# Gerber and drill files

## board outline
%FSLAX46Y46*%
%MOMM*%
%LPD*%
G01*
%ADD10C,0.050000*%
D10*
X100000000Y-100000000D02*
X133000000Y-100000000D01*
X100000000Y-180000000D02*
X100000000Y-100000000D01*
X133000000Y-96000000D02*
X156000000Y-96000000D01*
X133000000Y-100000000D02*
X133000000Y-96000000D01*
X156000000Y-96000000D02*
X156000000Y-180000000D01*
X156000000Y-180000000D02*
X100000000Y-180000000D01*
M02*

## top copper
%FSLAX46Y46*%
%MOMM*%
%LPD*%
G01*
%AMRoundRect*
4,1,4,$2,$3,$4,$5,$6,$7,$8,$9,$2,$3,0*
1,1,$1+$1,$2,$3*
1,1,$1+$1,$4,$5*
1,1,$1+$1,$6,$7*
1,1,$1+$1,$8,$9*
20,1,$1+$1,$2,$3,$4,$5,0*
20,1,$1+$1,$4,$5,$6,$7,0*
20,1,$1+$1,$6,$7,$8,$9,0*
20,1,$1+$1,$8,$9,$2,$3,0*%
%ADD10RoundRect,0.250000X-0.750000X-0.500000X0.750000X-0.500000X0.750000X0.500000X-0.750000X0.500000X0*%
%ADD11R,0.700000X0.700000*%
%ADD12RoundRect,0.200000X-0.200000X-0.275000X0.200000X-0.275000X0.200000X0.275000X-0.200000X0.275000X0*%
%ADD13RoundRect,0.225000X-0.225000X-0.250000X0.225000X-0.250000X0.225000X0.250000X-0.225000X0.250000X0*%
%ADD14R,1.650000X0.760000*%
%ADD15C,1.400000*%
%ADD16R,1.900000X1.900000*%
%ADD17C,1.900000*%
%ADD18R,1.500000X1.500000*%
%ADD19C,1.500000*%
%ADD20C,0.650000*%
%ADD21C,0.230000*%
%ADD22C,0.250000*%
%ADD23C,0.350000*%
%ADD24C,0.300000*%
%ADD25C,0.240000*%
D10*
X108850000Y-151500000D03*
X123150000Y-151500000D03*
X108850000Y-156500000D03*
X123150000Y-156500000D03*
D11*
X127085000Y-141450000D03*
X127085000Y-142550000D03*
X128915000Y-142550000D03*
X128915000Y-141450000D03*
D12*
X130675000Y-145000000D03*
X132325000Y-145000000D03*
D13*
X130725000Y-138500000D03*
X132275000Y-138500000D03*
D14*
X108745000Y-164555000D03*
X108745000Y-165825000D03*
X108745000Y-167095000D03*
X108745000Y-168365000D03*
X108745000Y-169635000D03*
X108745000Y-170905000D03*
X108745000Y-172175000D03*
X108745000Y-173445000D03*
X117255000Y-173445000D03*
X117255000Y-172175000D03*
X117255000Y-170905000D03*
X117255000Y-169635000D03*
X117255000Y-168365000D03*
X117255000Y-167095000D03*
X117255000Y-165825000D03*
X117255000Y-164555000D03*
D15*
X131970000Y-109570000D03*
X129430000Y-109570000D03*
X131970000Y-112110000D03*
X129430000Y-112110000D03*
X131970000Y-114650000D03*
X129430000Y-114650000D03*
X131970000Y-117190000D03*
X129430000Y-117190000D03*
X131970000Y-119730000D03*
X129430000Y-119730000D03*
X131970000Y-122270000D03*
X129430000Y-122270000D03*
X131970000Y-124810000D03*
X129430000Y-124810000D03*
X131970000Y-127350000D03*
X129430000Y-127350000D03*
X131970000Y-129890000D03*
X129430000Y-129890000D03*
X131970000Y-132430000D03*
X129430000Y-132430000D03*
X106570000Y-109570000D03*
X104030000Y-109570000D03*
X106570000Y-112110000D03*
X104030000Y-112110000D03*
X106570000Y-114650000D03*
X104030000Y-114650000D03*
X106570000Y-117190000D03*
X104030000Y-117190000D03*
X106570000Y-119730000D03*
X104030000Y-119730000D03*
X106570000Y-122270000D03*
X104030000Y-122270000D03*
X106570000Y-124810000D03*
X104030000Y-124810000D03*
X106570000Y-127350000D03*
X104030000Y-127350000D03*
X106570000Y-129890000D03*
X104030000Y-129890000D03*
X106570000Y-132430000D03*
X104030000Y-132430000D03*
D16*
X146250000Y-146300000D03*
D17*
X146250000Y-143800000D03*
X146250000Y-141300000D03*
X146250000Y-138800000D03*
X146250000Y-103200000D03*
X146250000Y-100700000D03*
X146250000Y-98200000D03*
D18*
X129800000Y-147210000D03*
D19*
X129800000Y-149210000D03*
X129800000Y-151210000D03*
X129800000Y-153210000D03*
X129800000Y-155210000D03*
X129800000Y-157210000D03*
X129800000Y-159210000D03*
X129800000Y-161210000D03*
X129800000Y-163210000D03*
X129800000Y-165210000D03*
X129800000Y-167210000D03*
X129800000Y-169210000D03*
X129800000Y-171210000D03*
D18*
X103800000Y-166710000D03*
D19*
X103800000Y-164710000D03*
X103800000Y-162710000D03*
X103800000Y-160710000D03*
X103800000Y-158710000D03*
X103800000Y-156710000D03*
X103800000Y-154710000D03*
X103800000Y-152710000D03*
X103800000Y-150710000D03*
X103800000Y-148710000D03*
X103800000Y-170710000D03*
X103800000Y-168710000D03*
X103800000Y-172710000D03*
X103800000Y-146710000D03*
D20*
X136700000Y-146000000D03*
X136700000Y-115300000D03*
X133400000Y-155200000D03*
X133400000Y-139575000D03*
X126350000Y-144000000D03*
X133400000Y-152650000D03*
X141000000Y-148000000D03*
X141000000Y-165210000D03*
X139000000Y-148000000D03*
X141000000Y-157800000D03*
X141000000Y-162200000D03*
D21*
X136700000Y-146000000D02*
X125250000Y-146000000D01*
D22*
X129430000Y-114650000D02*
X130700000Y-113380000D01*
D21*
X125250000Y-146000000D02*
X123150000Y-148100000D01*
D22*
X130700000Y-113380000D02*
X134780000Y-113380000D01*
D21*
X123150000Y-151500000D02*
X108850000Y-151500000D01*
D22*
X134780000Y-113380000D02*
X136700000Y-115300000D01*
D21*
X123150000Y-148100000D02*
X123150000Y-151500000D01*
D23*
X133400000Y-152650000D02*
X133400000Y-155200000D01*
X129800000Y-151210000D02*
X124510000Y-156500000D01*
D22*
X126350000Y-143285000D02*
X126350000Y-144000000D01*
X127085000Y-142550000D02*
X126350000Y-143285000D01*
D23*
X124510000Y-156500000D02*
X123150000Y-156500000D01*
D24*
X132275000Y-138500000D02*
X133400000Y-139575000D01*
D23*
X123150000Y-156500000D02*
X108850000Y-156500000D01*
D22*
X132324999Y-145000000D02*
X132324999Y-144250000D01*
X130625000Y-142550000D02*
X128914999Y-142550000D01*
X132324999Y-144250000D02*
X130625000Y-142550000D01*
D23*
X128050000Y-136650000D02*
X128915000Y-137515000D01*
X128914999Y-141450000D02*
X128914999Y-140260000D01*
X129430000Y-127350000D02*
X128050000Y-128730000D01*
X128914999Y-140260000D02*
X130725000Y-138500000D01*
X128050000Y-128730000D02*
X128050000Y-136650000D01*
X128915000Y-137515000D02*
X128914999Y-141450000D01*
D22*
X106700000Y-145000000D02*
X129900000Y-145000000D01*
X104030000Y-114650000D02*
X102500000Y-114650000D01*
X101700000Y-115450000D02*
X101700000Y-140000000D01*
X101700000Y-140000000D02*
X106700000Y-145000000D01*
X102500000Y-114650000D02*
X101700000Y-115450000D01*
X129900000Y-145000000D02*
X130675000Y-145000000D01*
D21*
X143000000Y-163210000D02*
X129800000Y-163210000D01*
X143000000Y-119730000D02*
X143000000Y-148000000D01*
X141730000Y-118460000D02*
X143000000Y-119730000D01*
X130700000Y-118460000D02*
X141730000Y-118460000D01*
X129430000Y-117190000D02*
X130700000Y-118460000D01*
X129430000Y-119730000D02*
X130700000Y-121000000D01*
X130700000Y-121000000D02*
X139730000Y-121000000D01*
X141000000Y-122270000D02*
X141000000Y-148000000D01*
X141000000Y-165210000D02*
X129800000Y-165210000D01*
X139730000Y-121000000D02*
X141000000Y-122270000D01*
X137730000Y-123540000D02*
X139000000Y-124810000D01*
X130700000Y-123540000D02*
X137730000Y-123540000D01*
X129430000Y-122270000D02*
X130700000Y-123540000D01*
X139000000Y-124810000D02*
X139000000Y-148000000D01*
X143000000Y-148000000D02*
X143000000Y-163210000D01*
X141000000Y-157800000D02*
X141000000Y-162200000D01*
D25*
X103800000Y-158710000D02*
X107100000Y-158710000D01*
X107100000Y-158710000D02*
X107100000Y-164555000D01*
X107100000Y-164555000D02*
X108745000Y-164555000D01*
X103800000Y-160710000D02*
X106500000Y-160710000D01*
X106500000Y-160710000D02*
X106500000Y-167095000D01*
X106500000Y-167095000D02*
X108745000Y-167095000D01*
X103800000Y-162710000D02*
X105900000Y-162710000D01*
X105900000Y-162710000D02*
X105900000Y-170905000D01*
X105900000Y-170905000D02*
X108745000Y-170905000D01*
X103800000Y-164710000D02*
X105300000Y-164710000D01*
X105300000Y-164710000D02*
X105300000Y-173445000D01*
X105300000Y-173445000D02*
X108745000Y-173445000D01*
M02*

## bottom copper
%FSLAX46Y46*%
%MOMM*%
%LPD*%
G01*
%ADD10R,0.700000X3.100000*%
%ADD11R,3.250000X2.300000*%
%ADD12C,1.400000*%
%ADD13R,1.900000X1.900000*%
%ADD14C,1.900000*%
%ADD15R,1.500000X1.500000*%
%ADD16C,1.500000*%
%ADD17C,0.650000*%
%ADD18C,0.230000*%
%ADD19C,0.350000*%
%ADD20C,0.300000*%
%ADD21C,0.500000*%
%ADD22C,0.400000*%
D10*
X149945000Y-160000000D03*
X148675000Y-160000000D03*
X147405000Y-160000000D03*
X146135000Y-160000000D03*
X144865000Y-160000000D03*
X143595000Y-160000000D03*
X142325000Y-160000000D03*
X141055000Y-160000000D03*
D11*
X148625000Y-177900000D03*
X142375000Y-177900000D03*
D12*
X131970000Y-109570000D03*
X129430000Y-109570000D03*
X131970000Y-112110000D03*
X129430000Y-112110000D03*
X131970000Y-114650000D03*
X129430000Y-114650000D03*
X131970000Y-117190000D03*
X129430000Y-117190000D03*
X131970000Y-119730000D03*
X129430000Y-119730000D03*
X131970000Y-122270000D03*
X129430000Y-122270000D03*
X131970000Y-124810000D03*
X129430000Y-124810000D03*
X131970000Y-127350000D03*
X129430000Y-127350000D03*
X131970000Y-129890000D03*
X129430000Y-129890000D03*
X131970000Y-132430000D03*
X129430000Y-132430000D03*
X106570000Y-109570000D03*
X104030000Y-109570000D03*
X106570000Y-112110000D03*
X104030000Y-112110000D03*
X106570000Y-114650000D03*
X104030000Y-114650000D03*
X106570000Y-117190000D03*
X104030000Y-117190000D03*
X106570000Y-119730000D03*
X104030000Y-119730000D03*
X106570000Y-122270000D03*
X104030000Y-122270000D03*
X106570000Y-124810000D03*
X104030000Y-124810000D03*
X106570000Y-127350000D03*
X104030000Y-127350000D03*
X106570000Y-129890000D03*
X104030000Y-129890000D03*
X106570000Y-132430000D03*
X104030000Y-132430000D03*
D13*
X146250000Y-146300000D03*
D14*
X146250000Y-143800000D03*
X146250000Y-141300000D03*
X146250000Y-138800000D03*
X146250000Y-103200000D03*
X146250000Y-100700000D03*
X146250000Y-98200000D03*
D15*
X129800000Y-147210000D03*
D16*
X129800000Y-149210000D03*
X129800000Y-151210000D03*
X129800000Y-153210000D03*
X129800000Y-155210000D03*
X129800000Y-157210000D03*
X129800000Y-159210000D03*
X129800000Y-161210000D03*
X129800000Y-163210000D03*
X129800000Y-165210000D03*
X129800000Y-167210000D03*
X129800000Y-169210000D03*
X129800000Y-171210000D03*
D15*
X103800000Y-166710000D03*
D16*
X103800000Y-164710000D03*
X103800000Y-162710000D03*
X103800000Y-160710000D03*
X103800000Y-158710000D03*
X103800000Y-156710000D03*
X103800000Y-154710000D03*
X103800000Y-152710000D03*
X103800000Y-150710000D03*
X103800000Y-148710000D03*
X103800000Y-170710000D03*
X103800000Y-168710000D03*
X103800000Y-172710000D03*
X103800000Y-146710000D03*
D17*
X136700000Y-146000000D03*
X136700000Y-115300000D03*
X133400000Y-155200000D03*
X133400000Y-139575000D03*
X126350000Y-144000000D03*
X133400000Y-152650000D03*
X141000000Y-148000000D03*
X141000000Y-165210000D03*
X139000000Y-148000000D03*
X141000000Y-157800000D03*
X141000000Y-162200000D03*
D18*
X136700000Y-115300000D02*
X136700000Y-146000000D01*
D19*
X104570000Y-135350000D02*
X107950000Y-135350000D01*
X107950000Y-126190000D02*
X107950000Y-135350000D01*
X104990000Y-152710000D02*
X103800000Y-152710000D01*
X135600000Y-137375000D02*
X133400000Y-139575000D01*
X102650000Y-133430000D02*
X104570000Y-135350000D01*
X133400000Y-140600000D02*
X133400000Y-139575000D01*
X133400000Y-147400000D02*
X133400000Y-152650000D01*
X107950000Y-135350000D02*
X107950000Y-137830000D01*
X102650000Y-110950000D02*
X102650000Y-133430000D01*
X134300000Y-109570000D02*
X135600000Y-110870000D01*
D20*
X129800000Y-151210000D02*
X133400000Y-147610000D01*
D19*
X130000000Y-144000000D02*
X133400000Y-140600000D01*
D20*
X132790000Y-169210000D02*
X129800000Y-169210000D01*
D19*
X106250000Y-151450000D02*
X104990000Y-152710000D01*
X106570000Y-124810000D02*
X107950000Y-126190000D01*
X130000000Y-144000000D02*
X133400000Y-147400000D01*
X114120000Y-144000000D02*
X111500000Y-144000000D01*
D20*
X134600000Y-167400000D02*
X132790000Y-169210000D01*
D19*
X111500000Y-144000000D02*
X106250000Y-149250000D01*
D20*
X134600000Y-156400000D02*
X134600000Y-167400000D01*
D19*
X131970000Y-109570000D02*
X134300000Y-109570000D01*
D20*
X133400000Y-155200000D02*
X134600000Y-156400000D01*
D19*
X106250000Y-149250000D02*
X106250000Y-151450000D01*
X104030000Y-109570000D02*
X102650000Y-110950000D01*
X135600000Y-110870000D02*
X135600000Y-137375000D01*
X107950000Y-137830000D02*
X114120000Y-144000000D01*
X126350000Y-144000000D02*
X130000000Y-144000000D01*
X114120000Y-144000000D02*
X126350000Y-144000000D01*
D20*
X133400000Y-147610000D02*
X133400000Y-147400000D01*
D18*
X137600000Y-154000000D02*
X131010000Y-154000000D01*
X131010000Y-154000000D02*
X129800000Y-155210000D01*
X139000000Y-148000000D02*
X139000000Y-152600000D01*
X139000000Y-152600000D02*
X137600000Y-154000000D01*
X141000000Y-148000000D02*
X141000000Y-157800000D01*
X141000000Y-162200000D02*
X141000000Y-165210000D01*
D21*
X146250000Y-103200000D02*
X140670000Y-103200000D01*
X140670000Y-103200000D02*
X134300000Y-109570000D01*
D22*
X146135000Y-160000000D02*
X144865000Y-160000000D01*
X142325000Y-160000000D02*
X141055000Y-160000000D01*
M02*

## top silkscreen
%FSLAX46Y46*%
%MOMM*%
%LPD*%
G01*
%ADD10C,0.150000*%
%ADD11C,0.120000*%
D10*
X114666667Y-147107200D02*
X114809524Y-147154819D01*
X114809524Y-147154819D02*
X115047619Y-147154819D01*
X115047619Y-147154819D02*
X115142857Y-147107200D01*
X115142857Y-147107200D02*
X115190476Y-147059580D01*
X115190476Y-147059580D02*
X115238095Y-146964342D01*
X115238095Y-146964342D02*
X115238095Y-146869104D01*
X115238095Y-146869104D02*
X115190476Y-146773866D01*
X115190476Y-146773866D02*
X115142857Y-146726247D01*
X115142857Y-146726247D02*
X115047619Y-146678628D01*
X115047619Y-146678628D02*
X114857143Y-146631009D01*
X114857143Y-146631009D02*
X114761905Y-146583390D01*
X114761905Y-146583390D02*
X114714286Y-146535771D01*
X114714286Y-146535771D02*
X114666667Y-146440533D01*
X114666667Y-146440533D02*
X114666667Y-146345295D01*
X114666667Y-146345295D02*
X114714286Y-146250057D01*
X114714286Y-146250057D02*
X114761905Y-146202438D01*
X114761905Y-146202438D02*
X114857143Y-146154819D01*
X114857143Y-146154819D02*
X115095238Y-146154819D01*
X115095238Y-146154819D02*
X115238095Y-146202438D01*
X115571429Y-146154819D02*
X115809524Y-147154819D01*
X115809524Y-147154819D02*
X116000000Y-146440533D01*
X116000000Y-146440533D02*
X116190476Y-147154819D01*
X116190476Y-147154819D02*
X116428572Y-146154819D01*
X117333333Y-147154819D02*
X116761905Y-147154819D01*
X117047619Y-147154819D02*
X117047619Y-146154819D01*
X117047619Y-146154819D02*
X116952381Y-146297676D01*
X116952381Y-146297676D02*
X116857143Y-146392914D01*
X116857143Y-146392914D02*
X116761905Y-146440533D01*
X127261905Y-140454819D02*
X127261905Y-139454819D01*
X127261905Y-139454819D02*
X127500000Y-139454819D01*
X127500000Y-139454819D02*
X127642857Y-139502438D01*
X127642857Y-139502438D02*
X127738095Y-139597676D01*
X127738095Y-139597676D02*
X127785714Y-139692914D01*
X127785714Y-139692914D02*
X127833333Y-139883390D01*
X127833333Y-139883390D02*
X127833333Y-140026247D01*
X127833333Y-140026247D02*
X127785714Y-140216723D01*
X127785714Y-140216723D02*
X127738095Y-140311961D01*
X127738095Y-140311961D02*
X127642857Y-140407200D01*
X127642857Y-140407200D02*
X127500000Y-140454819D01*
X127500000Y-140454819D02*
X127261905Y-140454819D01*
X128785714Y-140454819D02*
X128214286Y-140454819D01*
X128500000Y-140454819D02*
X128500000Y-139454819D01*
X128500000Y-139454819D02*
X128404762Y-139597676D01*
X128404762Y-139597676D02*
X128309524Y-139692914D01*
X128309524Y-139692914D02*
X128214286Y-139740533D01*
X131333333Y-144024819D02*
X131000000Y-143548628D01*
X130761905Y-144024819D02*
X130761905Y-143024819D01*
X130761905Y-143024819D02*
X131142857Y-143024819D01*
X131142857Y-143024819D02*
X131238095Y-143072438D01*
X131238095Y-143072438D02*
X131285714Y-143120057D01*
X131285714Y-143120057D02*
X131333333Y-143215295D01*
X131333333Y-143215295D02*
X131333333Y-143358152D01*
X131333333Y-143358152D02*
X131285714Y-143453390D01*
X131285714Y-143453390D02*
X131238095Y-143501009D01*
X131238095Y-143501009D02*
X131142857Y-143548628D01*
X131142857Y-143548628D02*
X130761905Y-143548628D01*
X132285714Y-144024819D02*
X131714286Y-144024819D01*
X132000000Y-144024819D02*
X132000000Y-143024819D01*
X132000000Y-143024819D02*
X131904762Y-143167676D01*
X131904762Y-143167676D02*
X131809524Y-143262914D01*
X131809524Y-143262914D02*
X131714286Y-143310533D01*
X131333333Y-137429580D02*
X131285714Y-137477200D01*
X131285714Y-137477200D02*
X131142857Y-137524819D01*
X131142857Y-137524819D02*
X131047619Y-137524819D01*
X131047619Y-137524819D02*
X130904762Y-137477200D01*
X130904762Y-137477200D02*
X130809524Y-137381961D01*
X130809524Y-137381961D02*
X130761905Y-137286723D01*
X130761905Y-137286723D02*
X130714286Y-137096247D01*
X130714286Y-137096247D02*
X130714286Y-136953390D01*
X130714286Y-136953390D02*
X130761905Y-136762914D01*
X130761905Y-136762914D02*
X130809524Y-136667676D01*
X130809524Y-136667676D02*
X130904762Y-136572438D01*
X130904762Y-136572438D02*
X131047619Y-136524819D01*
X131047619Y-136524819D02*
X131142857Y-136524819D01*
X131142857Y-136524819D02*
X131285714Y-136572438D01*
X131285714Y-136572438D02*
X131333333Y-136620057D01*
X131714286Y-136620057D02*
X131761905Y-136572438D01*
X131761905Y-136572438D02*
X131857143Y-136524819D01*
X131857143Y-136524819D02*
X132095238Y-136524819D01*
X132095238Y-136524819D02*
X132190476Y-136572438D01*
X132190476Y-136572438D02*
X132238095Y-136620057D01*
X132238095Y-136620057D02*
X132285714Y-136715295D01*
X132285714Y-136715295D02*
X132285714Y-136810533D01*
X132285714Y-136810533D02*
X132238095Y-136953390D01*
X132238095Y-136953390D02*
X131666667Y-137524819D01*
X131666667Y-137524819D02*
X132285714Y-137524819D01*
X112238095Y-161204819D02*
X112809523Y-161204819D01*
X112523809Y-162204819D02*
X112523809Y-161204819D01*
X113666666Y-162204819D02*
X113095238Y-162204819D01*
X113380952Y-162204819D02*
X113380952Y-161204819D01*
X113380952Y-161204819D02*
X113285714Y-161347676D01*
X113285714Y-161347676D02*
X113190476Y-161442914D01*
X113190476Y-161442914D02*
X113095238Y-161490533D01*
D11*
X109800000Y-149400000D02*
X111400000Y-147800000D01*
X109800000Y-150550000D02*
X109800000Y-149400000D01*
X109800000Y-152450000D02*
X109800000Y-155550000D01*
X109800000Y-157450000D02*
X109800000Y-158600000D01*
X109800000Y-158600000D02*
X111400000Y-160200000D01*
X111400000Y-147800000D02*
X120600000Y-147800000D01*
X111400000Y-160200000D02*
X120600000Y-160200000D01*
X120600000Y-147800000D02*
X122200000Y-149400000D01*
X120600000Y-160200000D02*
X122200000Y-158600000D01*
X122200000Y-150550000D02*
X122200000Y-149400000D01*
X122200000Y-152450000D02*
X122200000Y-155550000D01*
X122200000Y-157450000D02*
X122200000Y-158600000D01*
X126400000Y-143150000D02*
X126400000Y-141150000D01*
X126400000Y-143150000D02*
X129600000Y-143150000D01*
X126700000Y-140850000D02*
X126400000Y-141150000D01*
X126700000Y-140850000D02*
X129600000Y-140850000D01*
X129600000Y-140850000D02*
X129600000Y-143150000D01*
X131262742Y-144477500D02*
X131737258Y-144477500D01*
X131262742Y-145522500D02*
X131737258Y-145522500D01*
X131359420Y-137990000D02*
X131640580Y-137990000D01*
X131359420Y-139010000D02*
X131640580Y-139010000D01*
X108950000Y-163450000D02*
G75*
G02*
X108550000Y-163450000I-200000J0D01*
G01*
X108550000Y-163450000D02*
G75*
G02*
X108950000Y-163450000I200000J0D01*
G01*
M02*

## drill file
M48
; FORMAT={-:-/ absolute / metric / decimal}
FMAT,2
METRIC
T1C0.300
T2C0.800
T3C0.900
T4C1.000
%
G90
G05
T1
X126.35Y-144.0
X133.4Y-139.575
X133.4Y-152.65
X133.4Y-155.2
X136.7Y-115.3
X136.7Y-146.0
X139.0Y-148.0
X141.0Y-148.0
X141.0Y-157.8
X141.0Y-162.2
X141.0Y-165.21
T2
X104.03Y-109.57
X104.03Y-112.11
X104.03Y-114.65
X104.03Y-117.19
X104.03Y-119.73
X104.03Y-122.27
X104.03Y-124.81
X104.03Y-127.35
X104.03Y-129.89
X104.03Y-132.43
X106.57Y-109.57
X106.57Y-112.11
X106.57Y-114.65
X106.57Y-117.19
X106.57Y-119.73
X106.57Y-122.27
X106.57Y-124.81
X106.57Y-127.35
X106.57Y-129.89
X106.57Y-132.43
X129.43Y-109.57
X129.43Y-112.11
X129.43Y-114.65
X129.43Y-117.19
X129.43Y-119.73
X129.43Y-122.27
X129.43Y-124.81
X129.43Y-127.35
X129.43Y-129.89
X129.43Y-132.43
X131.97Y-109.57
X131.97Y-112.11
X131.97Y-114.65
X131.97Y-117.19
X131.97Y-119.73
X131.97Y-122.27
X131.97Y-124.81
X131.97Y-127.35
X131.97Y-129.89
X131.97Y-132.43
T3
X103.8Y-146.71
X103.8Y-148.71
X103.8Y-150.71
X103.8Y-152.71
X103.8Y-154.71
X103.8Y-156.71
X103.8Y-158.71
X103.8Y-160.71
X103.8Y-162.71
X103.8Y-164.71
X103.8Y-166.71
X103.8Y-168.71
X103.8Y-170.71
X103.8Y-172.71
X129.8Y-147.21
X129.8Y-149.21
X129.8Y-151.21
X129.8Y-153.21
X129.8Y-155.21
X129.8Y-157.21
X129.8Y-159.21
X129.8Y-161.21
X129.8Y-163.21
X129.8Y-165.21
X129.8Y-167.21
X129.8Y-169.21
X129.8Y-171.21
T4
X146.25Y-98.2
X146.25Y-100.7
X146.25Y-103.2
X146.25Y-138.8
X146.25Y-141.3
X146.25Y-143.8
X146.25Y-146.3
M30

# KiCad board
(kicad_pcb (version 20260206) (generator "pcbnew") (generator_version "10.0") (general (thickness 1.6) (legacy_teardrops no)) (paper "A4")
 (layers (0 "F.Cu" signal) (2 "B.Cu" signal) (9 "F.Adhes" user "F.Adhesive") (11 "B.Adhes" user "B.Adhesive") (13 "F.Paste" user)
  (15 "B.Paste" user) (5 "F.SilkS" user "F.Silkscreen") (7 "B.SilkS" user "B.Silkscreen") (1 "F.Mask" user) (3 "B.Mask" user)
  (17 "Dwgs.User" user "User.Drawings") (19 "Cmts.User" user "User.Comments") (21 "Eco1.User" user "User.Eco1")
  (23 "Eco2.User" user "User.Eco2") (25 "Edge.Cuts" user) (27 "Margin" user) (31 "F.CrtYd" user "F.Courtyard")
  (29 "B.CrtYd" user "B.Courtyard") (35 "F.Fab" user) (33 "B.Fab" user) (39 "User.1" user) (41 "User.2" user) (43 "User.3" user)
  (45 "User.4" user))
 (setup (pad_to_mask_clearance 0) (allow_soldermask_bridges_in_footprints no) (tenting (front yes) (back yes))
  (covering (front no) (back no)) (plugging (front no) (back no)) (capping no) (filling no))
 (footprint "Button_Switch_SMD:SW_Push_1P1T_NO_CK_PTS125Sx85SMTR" (layer "F.Cu") (at 116 154)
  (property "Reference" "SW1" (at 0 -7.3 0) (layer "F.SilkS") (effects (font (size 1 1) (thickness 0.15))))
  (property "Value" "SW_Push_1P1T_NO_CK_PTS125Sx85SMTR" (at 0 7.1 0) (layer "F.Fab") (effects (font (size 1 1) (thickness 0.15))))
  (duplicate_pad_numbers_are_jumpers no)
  (fp_line (start -6.2 -4.6) (end -4.6 -6.2) (stroke (width 0.12) (type solid)) (layer "F.SilkS"))
  (fp_line (start -6.2 -3.45) (end -6.2 -4.6) (stroke (width 0.12) (type solid)) (layer "F.SilkS"))
  (fp_line (start -6.2 -1.55) (end -6.2 1.55) (stroke (width 0.12) (type solid)) (layer "F.SilkS"))
  (fp_line (start -6.2 3.45) (end -6.2 4.6) (stroke (width 0.12) (type solid)) (layer "F.SilkS"))
  (fp_line (start -6.2 4.6) (end -4.6 6.2) (stroke (width 0.12) (type solid)) (layer "F.SilkS"))
  (fp_line (start -4.6 -6.2) (end 4.6 -6.2) (stroke (width 0.12) (type solid)) (layer "F.SilkS"))
  (fp_line (start -4.6 6.2) (end 4.6 6.2) (stroke (width 0.12) (type solid)) (layer "F.SilkS"))
  (fp_line (start 4.6 -6.2) (end 6.2 -4.6) (stroke (width 0.12) (type solid)) (layer "F.SilkS"))
  (fp_line (start 4.6 6.2) (end 6.2 4.6) (stroke (width 0.12) (type solid)) (layer "F.SilkS"))
  (fp_line (start 6.2 -3.45) (end 6.2 -4.6) (stroke (width 0.12) (type solid)) (layer "F.SilkS"))
  (fp_line (start 6.2 -1.55) (end 6.2 1.55) (stroke (width 0.12) (type solid)) (layer "F.SilkS"))
  (fp_line (start 6.2 3.45) (end 6.2 4.6) (stroke (width 0.12) (type solid)) (layer "F.SilkS"))
  (pad "1" smd roundrect (at -7.15 -2.5) (size 2 1.5) (layers "F.Cu" "F.Mask" "F.Paste") (roundrect_rratio 0.1666666667)
   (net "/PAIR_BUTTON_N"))
  (pad "1" smd roundrect (at 7.15 -2.5) (size 2 1.5) (layers "F.Cu" "F.Mask" "F.Paste") (roundrect_rratio 0.1666666667)
   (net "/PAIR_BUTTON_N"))
  (pad "2" smd roundrect (at -7.15 2.5) (size 2 1.5) (layers "F.Cu" "F.Mask" "F.Paste") (roundrect_rratio 0.1666666667) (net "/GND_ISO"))
  (pad "2" smd roundrect (at 7.15 2.5) (size 2 1.5) (layers "F.Cu" "F.Mask" "F.Paste") (roundrect_rratio 0.1666666667) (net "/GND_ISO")))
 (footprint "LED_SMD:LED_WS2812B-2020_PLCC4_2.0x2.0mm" (layer "F.Cu") (at 128 142)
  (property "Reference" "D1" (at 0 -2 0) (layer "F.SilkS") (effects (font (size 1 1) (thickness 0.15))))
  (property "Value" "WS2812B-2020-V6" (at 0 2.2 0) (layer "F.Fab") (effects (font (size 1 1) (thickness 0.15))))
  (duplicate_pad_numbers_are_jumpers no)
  (fp_line (start -1.6 1.15) (end -1.6 -0.85) (stroke (width 0.12) (type solid)) (layer "F.SilkS"))
  (fp_line (start -1.6 1.15) (end 1.6 1.15) (stroke (width 0.12) (type solid)) (layer "F.SilkS"))
  (fp_line (start -1.3 -1.15) (end -1.6 -0.85) (stroke (width 0.12) (type default)) (layer "F.SilkS"))
  (fp_line (start -1.3 -1.15) (end 1.6 -1.15) (stroke (width 0.12) (type solid)) (layer "F.SilkS"))
  (fp_line (start 1.6 -1.15) (end 1.6 1.15) (stroke (width 0.12) (type solid)) (layer "F.SilkS"))
  (pad "1" smd rect (at -0.915 -0.55) (size 0.7 0.7) (layers "F.Cu" "F.Mask" "F.Paste"))
  (pad "2" smd rect (at -0.915 0.55) (size 0.7 0.7) (layers "F.Cu" "F.Mask" "F.Paste") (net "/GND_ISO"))
  (pad "3" smd rect (at 0.915 0.55) (size 0.7 0.7) (layers "F.Cu" "F.Mask" "F.Paste") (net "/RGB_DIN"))
  (pad "4" smd rect (at 0.915 -0.55) (size 0.7 0.7) (layers "F.Cu" "F.Mask" "F.Paste") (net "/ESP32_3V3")))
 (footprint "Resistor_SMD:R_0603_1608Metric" (layer "F.Cu") (at 131.5 145)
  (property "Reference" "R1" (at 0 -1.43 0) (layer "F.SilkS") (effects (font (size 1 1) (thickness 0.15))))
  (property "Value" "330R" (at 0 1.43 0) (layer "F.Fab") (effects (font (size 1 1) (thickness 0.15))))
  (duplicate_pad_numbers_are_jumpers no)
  (fp_line (start -0.237258 -0.5225) (end 0.237258 -0.5225) (stroke (width 0.12) (type solid)) (layer "F.SilkS"))
  (fp_line (start -0.237258 0.5225) (end 0.237258 0.5225) (stroke (width 0.12) (type solid)) (layer "F.SilkS"))
  (pad "1" smd roundrect (at -0.825 0) (size 0.8 0.95) (layers "F.Cu" "F.Mask" "F.Paste") (roundrect_rratio 0.25) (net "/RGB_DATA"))
  (pad "2" smd roundrect (at 0.825 0) (size 0.8 0.95) (layers "F.Cu" "F.Mask" "F.Paste") (roundrect_rratio 0.25) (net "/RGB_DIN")))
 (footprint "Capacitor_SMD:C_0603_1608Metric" (layer "F.Cu") (at 131.5 138.5)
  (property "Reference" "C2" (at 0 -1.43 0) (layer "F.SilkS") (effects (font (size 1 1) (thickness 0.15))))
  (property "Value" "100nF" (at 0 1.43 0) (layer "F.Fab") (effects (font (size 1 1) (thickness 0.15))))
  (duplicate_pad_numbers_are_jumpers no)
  (fp_line (start -0.14058 -0.51) (end 0.14058 -0.51) (stroke (width 0.12) (type solid)) (layer "F.SilkS"))
  (fp_line (start -0.14058 0.51) (end 0.14058 0.51) (stroke (width 0.12) (type solid)) (layer "F.SilkS"))
  (pad "1" smd roundrect (at -0.775 0) (size 0.9 0.95) (layers "F.Cu" "F.Mask" "F.Paste") (roundrect_rratio 0.25) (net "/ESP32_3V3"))
  (pad "2" smd roundrect (at 0.775 0) (size 0.9 0.95) (layers "F.Cu" "F.Mask" "F.Paste") (roundrect_rratio 0.25) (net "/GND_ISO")))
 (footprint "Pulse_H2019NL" (layer "F.Cu") (at 113 169)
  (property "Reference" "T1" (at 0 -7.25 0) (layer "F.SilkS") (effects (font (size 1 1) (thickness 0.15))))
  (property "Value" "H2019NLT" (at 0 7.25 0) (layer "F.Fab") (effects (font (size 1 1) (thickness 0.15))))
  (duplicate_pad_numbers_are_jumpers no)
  (fp_circle (center -4.25 -5.55) (end -4.05 -5.55) (stroke (width 0.12) (type default)) (fill no) (layer "F.SilkS"))
  (pad "1" smd rect (at -4.255 -4.445) (size 1.65 0.76) (layers "F.Cu" "F.Mask" "F.Paste") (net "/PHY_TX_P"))
  (pad "2" smd rect (at -4.255 -3.175) (size 1.65 0.76) (layers "F.Cu" "F.Mask" "F.Paste"))
  (pad "3" smd rect (at -4.255 -1.905) (size 1.65 0.76) (layers "F.Cu" "F.Mask" "F.Paste") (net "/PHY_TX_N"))
  (pad "4" smd rect (at -4.255 -0.635) (size 1.65 0.76) (layers "F.Cu" "F.Mask" "F.Paste"))
  (pad "5" smd rect (at -4.255 0.635) (size 1.65 0.76) (layers "F.Cu" "F.Mask" "F.Paste"))
  (pad "6" smd rect (at -4.255 1.905) (size 1.65 0.76) (layers "F.Cu" "F.Mask" "F.Paste") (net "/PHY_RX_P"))
  (pad "7" smd rect (at -4.255 3.175) (size 1.65 0.76) (layers "F.Cu" "F.Mask" "F.Paste"))
  (pad "8" smd rect (at -4.255 4.445) (size 1.65 0.76) (layers "F.Cu" "F.Mask" "F.Paste") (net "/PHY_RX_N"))
  (pad "9" smd rect (at 4.255 4.445) (size 1.65 0.76) (layers "F.Cu" "F.Mask" "F.Paste") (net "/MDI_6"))
  (pad "10" smd rect (at 4.255 3.175) (size 1.65 0.76) (layers "F.Cu" "F.Mask" "F.Paste") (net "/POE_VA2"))
  (pad "11" smd rect (at 4.255 1.905) (size 1.65 0.76) (layers "F.Cu" "F.Mask" "F.Paste") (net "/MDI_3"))
  (pad "12" smd rect (at 4.255 0.635) (size 1.65 0.76) (layers "F.Cu" "F.Mask" "F.Paste"))
  (pad "13" smd rect (at 4.255 -0.635) (size 1.65 0.76) (layers "F.Cu" "F.Mask" "F.Paste"))
  (pad "14" smd rect (at 4.255 -1.905) (size 1.65 0.76) (layers "F.Cu" "F.Mask" "F.Paste") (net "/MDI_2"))
  (pad "15" smd rect (at 4.255 -3.175) (size 1.65 0.76) (layers "F.Cu" "F.Mask" "F.Paste") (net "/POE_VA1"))
  (pad "16" smd rect (at 4.255 -4.445) (size 1.65 0.76) (layers "F.Cu" "F.Mask" "F.Paste") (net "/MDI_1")))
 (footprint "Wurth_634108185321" (layer "B.Cu") (at 145.5 169.15 180)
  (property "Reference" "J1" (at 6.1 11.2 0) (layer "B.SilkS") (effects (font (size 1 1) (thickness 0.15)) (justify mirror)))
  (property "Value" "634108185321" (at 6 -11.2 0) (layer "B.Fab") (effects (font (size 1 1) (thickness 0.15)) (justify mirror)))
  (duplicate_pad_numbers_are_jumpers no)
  (pad "1" smd rect (at -4.445 9.15 180) (size 0.7 3.1) (layers "B.Cu" "B.Mask" "B.Paste") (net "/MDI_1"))
  (pad "2" smd rect (at -3.175 9.15 180) (size 0.7 3.1) (layers "B.Cu" "B.Mask" "B.Paste") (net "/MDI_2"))
  (pad "3" smd rect (at -1.905 9.15 180) (size 0.7 3.1) (layers "B.Cu" "B.Mask" "B.Paste") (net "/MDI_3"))
  (pad "4" smd rect (at -0.635 9.15 180) (size 0.7 3.1) (layers "B.Cu" "B.Mask" "B.Paste") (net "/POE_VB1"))
  (pad "5" smd rect (at 0.635 9.15 180) (size 0.7 3.1) (layers "B.Cu" "B.Mask" "B.Paste") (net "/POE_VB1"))
  (pad "6" smd rect (at 1.905 9.15 180) (size 0.7 3.1) (layers "B.Cu" "B.Mask" "B.Paste") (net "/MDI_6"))
  (pad "7" smd rect (at 3.175 9.15 180) (size 0.7 3.1) (layers "B.Cu" "B.Mask" "B.Paste") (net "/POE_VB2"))
  (pad "8" smd rect (at 4.445 9.15 180) (size 0.7 3.1) (layers "B.Cu" "B.Mask" "B.Paste") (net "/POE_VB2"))
  (pad "SH" smd rect (at -3.125 -8.75 180) (size 3.25 2.3) (layers "B.Cu" "B.Mask" "B.Paste"))
  (pad "SH" smd rect (at 3.125 -8.75 180) (size 3.25 2.3) (layers "B.Cu" "B.Mask" "B.Paste")))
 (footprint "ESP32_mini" (layer "B.Cu") (at 118 121 180)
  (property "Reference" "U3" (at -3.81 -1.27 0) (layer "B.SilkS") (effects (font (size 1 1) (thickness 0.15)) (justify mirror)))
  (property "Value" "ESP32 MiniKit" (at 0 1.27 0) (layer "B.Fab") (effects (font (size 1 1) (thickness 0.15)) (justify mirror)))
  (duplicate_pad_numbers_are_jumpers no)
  (pad "1" thru_hole circle (at -13.97 11.43 270) (size 1.4 1.4) (drill 0.8) (layers "*.Cu" "*.Mask") (remove_unused_layers no)
   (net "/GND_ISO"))
  (pad "2" thru_hole circle (at -11.43 11.43 270) (size 1.4 1.4) (drill 0.8) (layers "*.Cu" "*.Mask") (remove_unused_layers no))
  (pad "3" thru_hole circle (at -13.97 8.89 270) (size 1.4 1.4) (drill 0.8) (layers "*.Cu" "*.Mask") (remove_unused_layers no))
  (pad "4" thru_hole circle (at -11.43 8.89 270) (size 1.4 1.4) (drill 0.8) (layers "*.Cu" "*.Mask") (remove_unused_layers no))
  (pad "5" thru_hole circle (at -13.97 6.35 270) (size 1.4 1.4) (drill 0.8) (layers "*.Cu" "*.Mask") (remove_unused_layers no))
  (pad "6" thru_hole circle (at -11.43 6.35 270) (size 1.4 1.4) (drill 0.8) (layers "*.Cu" "*.Mask") (remove_unused_layers no)
   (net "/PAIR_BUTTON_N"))
  (pad "7" thru_hole circle (at -13.97 3.81 270) (size 1.4 1.4) (drill 0.8) (layers "*.Cu" "*.Mask") (remove_unused_layers no))
  (pad "8" thru_hole circle (at -11.43 3.81 270) (size 1.4 1.4) (drill 0.8) (layers "*.Cu" "*.Mask") (remove_unused_layers no)
   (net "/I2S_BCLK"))
  (pad "9" thru_hole circle (at -13.97 1.27 270) (size 1.4 1.4) (drill 0.8) (layers "*.Cu" "*.Mask") (remove_unused_layers no))
  (pad "10" thru_hole circle (at -11.43 1.27 270) (size 1.4 1.4) (drill 0.8) (layers "*.Cu" "*.Mask") (remove_unused_layers no)
   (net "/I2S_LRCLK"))
  (pad "11" thru_hole circle (at -13.97 -1.27 270) (size 1.4 1.4) (drill 0.8) (layers "*.Cu" "*.Mask") (remove_unused_layers no))
  (pad "12" thru_hole circle (at -11.43 -1.27 270) (size 1.4 1.4) (drill 0.8) (layers "*.Cu" "*.Mask") (remove_unused_layers no)
   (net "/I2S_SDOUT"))
  (pad "13" thru_hole circle (at -13.97 -3.81 270) (size 1.4 1.4) (drill 0.8) (layers "*.Cu" "*.Mask") (remove_unused_layers no))
  (pad "14" thru_hole circle (at -11.43 -3.81 270) (size 1.4 1.4) (drill 0.8) (layers "*.Cu" "*.Mask") (remove_unused_layers no))
  (pad "15" thru_hole circle (at -13.97 -6.35 270) (size 1.4 1.4) (drill 0.8) (layers "*.Cu" "*.Mask") (remove_unused_layers no))
  (pad "16" thru_hole circle (at -11.43 -6.35 270) (size 1.4 1.4) (drill 0.8) (layers "*.Cu" "*.Mask") (remove_unused_layers no)
   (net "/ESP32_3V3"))
  (pad "17" thru_hole circle (at -13.97 -8.89 270) (size 1.4 1.4) (drill 0.8) (layers "*.Cu" "*.Mask") (remove_unused_layers no))
  (pad "18" thru_hole circle (at -11.43 -8.89 270) (size 1.4 1.4) (drill 0.8) (layers "*.Cu" "*.Mask") (remove_unused_layers no))
  (pad "19" thru_hole circle (at -13.97 -11.43 270) (size 1.4 1.4) (drill 0.8) (layers "*.Cu" "*.Mask") (remove_unused_layers no))
  (pad "20" thru_hole circle (at -11.43 -11.43 270) (size 1.4 1.4) (drill 0.8) (layers "*.Cu" "*.Mask") (remove_unused_layers no))
  (pad "21" thru_hole circle (at 11.43 11.43 270) (size 1.4 1.4) (drill 0.8) (layers "*.Cu" "*.Mask") (remove_unused_layers no))
  (pad "22" thru_hole circle (at 13.97 11.43 270) (size 1.4 1.4) (drill 0.8) (layers "*.Cu" "*.Mask") (remove_unused_layers no)
   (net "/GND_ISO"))
  (pad "23" thru_hole circle (at 11.43 8.89 270) (size 1.4 1.4) (drill 0.8) (layers "*.Cu" "*.Mask") (remove_unused_layers no))
  (pad "24" thru_hole circle (at 13.97 8.89 270) (size 1.4 1.4) (drill 0.8) (layers "*.Cu" "*.Mask") (remove_unused_layers no))
  (pad "25" thru_hole circle (at 11.43 6.35 270) (size 1.4 1.4) (drill 0.8) (layers "*.Cu" "*.Mask") (remove_unused_layers no))
  (pad "26" thru_hole circle (at 13.97 6.35 270) (size 1.4 1.4) (drill 0.8) (layers "*.Cu" "*.Mask") (remove_unused_layers no)
   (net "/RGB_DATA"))
  (pad "27" thru_hole circle (at 11.43 3.81 270) (size 1.4 1.4) (drill 0.8) (layers "*.Cu" "*.Mask") (remove_unused_layers no))
  (pad "28" thru_hole circle (at 13.97 3.81 270) (size 1.4 1.4) (drill 0.8) (layers "*.Cu" "*.Mask") (remove_unused_layers no))
  (pad "29" thru_hole circle (at 11.43 1.27 270) (size 1.4 1.4) (drill 0.8) (layers "*.Cu" "*.Mask") (remove_unused_layers no))
  (pad "30" thru_hole circle (at 13.97 1.27 270) (size 1.4 1.4) (drill 0.8) (layers "*.Cu" "*.Mask") (remove_unused_layers no))
  (pad "31" thru_hole circle (at 11.43 -1.27 270) (size 1.4 1.4) (drill 0.8) (layers "*.Cu" "*.Mask") (remove_unused_layers no))
  (pad "32" thru_hole circle (at 13.97 -1.27 270) (size 1.4 1.4) (drill 0.8) (layers "*.Cu" "*.Mask") (remove_unused_layers no))
  (pad "33" thru_hole circle (at 11.43 -3.81 270) (size 1.4 1.4) (drill 0.8) (layers "*.Cu" "*.Mask") (remove_unused_layers no)
   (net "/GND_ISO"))
  (pad "34" thru_hole circle (at 13.97 -3.81 270) (size 1.4 1.4) (drill 0.8) (layers "*.Cu" "*.Mask") (remove_unused_layers no))
  (pad "35" thru_hole circle (at 11.43 -6.35 270) (size 1.4 1.4) (drill 0.8) (layers "*.Cu" "*.Mask") (remove_unused_layers no))
  (pad "36" thru_hole circle (at 13.97 -6.35 270) (size 1.4 1.4) (drill 0.8) (layers "*.Cu" "*.Mask") (remove_unused_layers no))
  (pad "37" thru_hole circle (at 11.43 -8.89 270) (size 1.4 1.4) (drill 0.8) (layers "*.Cu" "*.Mask") (remove_unused_layers no))
  (pad "38" thru_hole circle (at 13.97 -8.89 270) (size 1.4 1.4) (drill 0.8) (layers "*.Cu" "*.Mask") (remove_unused_layers no))
  (pad "39" thru_hole circle (at 11.43 -11.43 270) (size 1.4 1.4) (drill 0.8) (layers "*.Cu" "*.Mask") (remove_unused_layers no))
  (pad "40" thru_hole circle (at 13.97 -11.43 270) (size 1.4 1.4) (drill 0.8) (layers "*.Cu" "*.Mask") (remove_unused_layers no)))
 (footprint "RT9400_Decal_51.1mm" (layer "B.Cu") (at 146.25 146.3 90)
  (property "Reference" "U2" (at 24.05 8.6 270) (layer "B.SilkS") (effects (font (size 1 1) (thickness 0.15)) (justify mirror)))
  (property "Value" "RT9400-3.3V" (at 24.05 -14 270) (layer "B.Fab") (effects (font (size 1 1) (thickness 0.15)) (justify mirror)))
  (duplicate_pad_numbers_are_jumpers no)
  (pad "1" thru_hole rect (at 0 0 90) (size 1.9 1.9) (drill 1) (layers "*.Cu" "*.Mask") (remove_unused_layers no) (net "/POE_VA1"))
  (pad "2" thru_hole circle (at 2.5 0 90) (size 1.9 1.9) (drill 1) (layers "*.Cu" "*.Mask") (remove_unused_layers no) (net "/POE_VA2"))
  (pad "3" thru_hole circle (at 5 0 90) (size 1.9 1.9) (drill 1) (layers "*.Cu" "*.Mask") (remove_unused_layers no) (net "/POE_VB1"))
  (pad "4" thru_hole circle (at 7.5 0 90) (size 1.9 1.9) (drill 1) (layers "*.Cu" "*.Mask") (remove_unused_layers no) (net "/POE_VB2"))
  (pad "5" thru_hole circle (at 43.1 0 90) (size 1.9 1.9) (drill 1) (layers "*.Cu" "*.Mask") (remove_unused_layers no) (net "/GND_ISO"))
  (pad "6" thru_hole circle (at 45.6 0 90) (size 1.9 1.9) (drill 1) (layers "*.Cu" "*.Mask") (remove_unused_layers no) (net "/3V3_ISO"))
  (pad "7" thru_hole circle (at 48.1 0 90) (size 1.9 1.9) (drill 1) (layers "*.Cu" "*.Mask") (remove_unused_layers no)))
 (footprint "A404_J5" (layer "B.Cu") (at 131 145.5 180)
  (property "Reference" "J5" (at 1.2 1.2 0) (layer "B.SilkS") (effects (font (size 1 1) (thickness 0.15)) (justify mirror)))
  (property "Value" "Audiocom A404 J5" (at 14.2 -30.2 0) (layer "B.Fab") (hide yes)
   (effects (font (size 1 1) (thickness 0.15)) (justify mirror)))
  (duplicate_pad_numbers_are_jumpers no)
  (pad "1" thru_hole rect (at 1.2 -1.71 180) (size 1.5 1.5) (drill 0.9) (layers "*.Cu" "*.Mask") (remove_unused_layers no))
  (pad "2" thru_hole circle (at 1.2 -3.71 180) (size 1.5 1.5) (drill 0.9) (layers "*.Cu" "*.Mask") (remove_unused_layers no))
  (pad "3" thru_hole circle (at 1.2 -5.71 180) (size 1.5 1.5) (drill 0.9) (layers "*.Cu" "*.Mask") (remove_unused_layers no)
   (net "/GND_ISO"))
  (pad "4" thru_hole circle (at 1.2 -7.71 180) (size 1.5 1.5) (drill 0.9) (layers "*.Cu" "*.Mask") (remove_unused_layers no))
  (pad "5" thru_hole circle (at 1.2 -9.71 180) (size 1.5 1.5) (drill 0.9) (layers "*.Cu" "*.Mask") (remove_unused_layers no)
   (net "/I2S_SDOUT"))
  (pad "6" thru_hole circle (at 1.2 -11.71 180) (size 1.5 1.5) (drill 0.9) (layers "*.Cu" "*.Mask") (remove_unused_layers no))
  (pad "7" thru_hole circle (at 1.2 -13.71 180) (size 1.5 1.5) (drill 0.9) (layers "*.Cu" "*.Mask") (remove_unused_layers no))
  (pad "8" thru_hole circle (at 1.2 -15.71 180) (size 1.5 1.5) (drill 0.9) (layers "*.Cu" "*.Mask") (remove_unused_layers no))
  (pad "9" thru_hole circle (at 1.2 -17.71 180) (size 1.5 1.5) (drill 0.9) (layers "*.Cu" "*.Mask") (remove_unused_layers no)
   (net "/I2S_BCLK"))
  (pad "10" thru_hole circle (at 1.2 -19.71 180) (size 1.5 1.5) (drill 0.9) (layers "*.Cu" "*.Mask") (remove_unused_layers no)
   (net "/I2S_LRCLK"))
  (pad "11" thru_hole circle (at 1.2 -21.71 180) (size 1.5 1.5) (drill 0.9) (layers "*.Cu" "*.Mask") (remove_unused_layers no))
  (pad "12" thru_hole circle (at 1.2 -23.71 180) (size 1.5 1.5) (drill 0.9) (layers "*.Cu" "*.Mask") (remove_unused_layers no)
   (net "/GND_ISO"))
  (pad "13" thru_hole circle (at 1.2 -25.71 180) (size 1.5 1.5) (drill 0.9) (layers "*.Cu" "*.Mask") (remove_unused_layers no)))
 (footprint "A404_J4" (layer "B.Cu") (at 131 145.5 180)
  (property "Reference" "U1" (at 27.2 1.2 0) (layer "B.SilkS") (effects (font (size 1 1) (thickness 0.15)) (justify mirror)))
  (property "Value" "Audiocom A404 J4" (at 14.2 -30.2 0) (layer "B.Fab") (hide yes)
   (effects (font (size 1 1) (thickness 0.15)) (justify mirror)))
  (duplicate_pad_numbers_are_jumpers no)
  (pad "1" thru_hole rect (at 27.2 -21.21 180) (size 1.5 1.5) (drill 0.9) (layers "*.Cu" "*.Mask") (remove_unused_layers no))
  (pad "2" thru_hole circle (at 27.2 -19.21 180) (size 1.5 1.5) (drill 0.9) (layers "*.Cu" "*.Mask") (remove_unused_layers no)
   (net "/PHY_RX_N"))
  (pad "3" thru_hole circle (at 27.2 -17.21 180) (size 1.5 1.5) (drill 0.9) (layers "*.Cu" "*.Mask") (remove_unused_layers no)
   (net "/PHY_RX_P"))
  (pad "4" thru_hole circle (at 27.2 -15.21 180) (size 1.5 1.5) (drill 0.9) (layers "*.Cu" "*.Mask") (remove_unused_layers no)
   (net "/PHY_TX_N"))
  (pad "5" thru_hole circle (at 27.2 -13.21 180) (size 1.5 1.5) (drill 0.9) (layers "*.Cu" "*.Mask") (remove_unused_layers no)
   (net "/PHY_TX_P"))
  (pad "6" thru_hole circle (at 27.2 -11.21 180) (size 1.5 1.5) (drill 0.9) (layers "*.Cu" "*.Mask") (remove_unused_layers no))
  (pad "7" thru_hole circle (at 27.2 -9.21 180) (size 1.5 1.5) (drill 0.9) (layers "*.Cu" "*.Mask") (remove_unused_layers no)
   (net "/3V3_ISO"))
  (pad "8" thru_hole circle (at 27.2 -7.21 180) (size 1.5 1.5) (drill 0.9) (layers "*.Cu" "*.Mask") (remove_unused_layers no)
   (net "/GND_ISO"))
  (pad "9" thru_hole circle (at 27.2 -5.21 180) (size 1.5 1.5) (drill 0.9) (layers "*.Cu" "*.Mask") (remove_unused_layers no))
  (pad "10" thru_hole circle (at 27.2 -3.21 180) (size 1.5 1.5) (drill 0.9) (layers "*.Cu" "*.Mask") (remove_unused_layers no))
  (pad "11" thru_hole circle (at 27.2 -25.21 180) (size 1.5 1.5) (drill 0.9) (layers "*.Cu" "*.Mask") (remove_unused_layers no))
  (pad "12" thru_hole circle (at 27.2 -23.21 180) (size 1.5 1.5) (drill 0.9) (layers "*.Cu" "*.Mask") (remove_unused_layers no))
  (pad "13" thru_hole circle (at 27.2 -27.21 180) (size 1.5 1.5) (drill 0.9) (layers "*.Cu" "*.Mask") (remove_unused_layers no))
  (pad "14" thru_hole circle (at 27.2 -1.21 180) (size 1.5 1.5) (drill 0.9) (layers "*.Cu" "*.Mask") (remove_unused_layers no)))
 (gr_line (start 100 100) (end 133 100) (stroke (width 0.05) (type default)) (layer "Edge.Cuts"))
 (gr_line (start 100 180) (end 100 100) (stroke (width 0.05) (type default)) (layer "Edge.Cuts"))
 (gr_line (start 133 96) (end 156 96) (stroke (width 0.05) (type default)) (layer "Edge.Cuts"))
 (gr_line (start 133 100) (end 133 96) (stroke (width 0.05) (type default)) (layer "Edge.Cuts"))
 (gr_line (start 156 96) (end 156 180) (stroke (width 0.05) (type default)) (layer "Edge.Cuts"))
 (gr_line (start 156 180) (end 100 180) (stroke (width 0.05) (type default)) (layer "Edge.Cuts"))
 (segment (start 136.7 146) (end 125.25 146) (width 0.23) (layer "F.Cu") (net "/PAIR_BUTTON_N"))
 (segment (start 129.43 114.65) (end 130.7 113.38) (width 0.25) (layer "F.Cu") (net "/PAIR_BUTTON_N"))
 (segment (start 125.25 146) (end 123.15 148.1) (width 0.23) (layer "F.Cu") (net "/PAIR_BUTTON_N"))
 (segment (start 130.7 113.38) (end 134.78 113.38) (width 0.25) (layer "F.Cu") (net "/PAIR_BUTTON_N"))
 (segment (start 123.15 151.5) (end 108.85 151.5) (width 0.23) (layer "F.Cu") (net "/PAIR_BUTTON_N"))
 (segment (start 134.78 113.38) (end 136.7 115.3) (width 0.25) (layer "F.Cu") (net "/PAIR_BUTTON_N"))
 (segment (start 123.15 148.1) (end 123.15 151.5) (width 0.23) (layer "F.Cu") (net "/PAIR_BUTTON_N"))
 (via (at 136.7 146) (size 0.65) (drill 0.3) (layers "F.Cu" "B.Cu") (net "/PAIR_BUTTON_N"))
 (via (at 136.7 115.3) (size 0.65) (drill 0.3) (layers "F.Cu" "B.Cu") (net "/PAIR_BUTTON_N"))
 (segment (start 136.7 115.3) (end 136.7 146) (width 0.23) (layer "B.Cu") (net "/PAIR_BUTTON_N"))
 (segment (start 133.4 152.65) (end 133.4 155.2) (width 0.35) (layer "F.Cu") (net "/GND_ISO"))
 (segment (start 129.8 151.21) (end 124.51 156.5) (width 0.35) (layer "F.Cu") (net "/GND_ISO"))
 (segment (start 126.35 143.285) (end 126.35 144) (width 0.25) (layer "F.Cu") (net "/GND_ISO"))
 (segment (start 127.085 142.55) (end 126.35 143.285) (width 0.25) (layer "F.Cu") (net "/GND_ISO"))
 (segment (start 124.51 156.5) (end 123.15 156.5) (width 0.35) (layer "F.Cu") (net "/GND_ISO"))
 (segment (start 132.275 138.5) (end 133.4 139.575) (width 0.3) (layer "F.Cu") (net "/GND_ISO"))
 (segment (start 123.15 156.5) (end 108.85 156.5) (width 0.35) (layer "F.Cu") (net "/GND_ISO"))
 (via (at 133.4 155.2) (size 0.65) (drill 0.3) (layers "F.Cu" "B.Cu") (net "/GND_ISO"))
 (via (at 133.4 139.575) (size 0.65) (drill 0.3) (layers "F.Cu" "B.Cu") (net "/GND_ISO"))
 (via (at 126.35 144) (size 0.65) (drill 0.3) (layers "F.Cu" "B.Cu") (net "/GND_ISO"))
 (via (at 133.4 152.65) (size 0.65) (drill 0.3) (layers "F.Cu" "B.Cu") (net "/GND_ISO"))
 (segment (start 104.57 135.35) (end 107.95 135.35) (width 0.35) (layer "B.Cu") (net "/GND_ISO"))
 (segment (start 107.95 126.19) (end 107.95 135.35) (width 0.35) (layer "B.Cu") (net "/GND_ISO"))
 (segment (start 104.99 152.71) (end 103.8 152.71) (width 0.35) (layer "B.Cu") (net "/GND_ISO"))
 (segment (start 135.6 137.375) (end 133.4 139.575) (width 0.35) (layer "B.Cu") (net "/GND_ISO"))
 (segment (start 102.65 133.43) (end 104.57 135.35) (width 0.35) (layer "B.Cu") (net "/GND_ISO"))
 (segment (start 133.4 140.6) (end 133.4 139.575) (width 0.35) (layer "B.Cu") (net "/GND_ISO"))
 (segment (start 133.4 147.4) (end 133.4 152.65) (width 0.35) (layer "B.Cu") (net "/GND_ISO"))
 (segment (start 107.95 135.35) (end 107.95 137.83) (width 0.35) (layer "B.Cu") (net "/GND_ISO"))
 (segment (start 102.65 110.95) (end 102.65 133.43) (width 0.35) (layer "B.Cu") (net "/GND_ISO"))
 (segment (start 134.3 109.57) (end 135.6 110.87) (width 0.35) (layer "B.Cu") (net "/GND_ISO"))
 (segment (start 129.8 151.21) (end 133.4 147.61) (width 0.3) (layer "B.Cu") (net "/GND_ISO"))
 (segment (start 130 144) (end 133.4 140.6) (width 0.35) (layer "B.Cu") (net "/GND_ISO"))
 (segment (start 132.79 169.21) (end 129.8 169.21) (width 0.3) (layer "B.Cu") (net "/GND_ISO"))
 (segment (start 106.25 151.45) (end 104.99 152.71) (width 0.35) (layer "B.Cu") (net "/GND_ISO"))
 (segment (start 106.57 124.81) (end 107.95 126.19) (width 0.35) (layer "B.Cu") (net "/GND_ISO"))
 (segment (start 130 144) (end 133.4 147.4) (width 0.35) (layer "B.Cu") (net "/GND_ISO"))
 (segment (start 114.12 144) (end 111.5 144) (width 0.35) (layer "B.Cu") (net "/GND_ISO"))
 (segment (start 134.6 167.4) (end 132.79 169.21) (width 0.3) (layer "B.Cu") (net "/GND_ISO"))
 (segment (start 111.5 144) (end 106.25 149.25) (width 0.35) (layer "B.Cu") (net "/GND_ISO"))
 (segment (start 134.6 156.4) (end 134.6 167.4) (width 0.3) (layer "B.Cu") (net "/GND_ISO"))
 (segment (start 131.97 109.57) (end 134.3 109.57) (width 0.35) (layer "B.Cu") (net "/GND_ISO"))
 (segment (start 133.4 155.2) (end 134.6 156.4) (width 0.3) (layer "B.Cu") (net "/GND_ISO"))
 (segment (start 106.25 149.25) (end 106.25 151.45) (width 0.35) (layer "B.Cu") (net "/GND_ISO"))
 (segment (start 104.03 109.57) (end 102.65 110.95) (width 0.35) (layer "B.Cu") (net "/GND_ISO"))
 (segment (start 135.6 110.87) (end 135.6 137.375) (width 0.35) (layer "B.Cu") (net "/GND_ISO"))
 (segment (start 107.95 137.83) (end 114.12 144) (width 0.35) (layer "B.Cu") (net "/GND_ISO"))
 (segment (start 126.35 144) (end 130 144) (width 0.35) (layer "B.Cu") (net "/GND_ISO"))
 (segment (start 114.12 144) (end 126.35 144) (width 0.35) (layer "B.Cu") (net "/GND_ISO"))
 (segment (start 133.4 147.61) (end 133.4 147.4) (width 0.3) (layer "B.Cu") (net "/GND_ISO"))
 (segment (start 132.324999 145) (end 132.324999 144.25) (width 0.25) (layer "F.Cu") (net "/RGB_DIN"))
 (segment (start 130.625 142.55) (end 128.914999 142.55) (width 0.25) (layer "F.Cu") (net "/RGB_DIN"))
 (segment (start 132.324999 144.25) (end 130.625 142.55) (width 0.25) (layer "F.Cu") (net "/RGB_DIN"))
 (segment (start 128.05 136.65) (end 128.915 137.515) (width 0.35) (layer "F.Cu") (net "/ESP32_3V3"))
 (segment (start 128.914999 141.45) (end 128.914999 140.26) (width 0.35) (layer "F.Cu") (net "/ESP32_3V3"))
 (segment (start 129.43 127.35) (end 128.05 128.73) (width 0.35) (layer "F.Cu") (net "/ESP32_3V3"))
 (segment (start 128.914999 140.26) (end 130.725 138.5) (width 0.35) (layer "F.Cu") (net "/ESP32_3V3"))
 (segment (start 128.05 128.73) (end 128.05 136.65) (width 0.35) (layer "F.Cu") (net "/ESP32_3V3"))
 (segment (start 128.915 137.515) (end 128.914999 141.45) (width 0.35) (layer "F.Cu") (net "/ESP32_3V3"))
 (segment (start 106.7 145) (end 129.9 145) (width 0.25) (layer "F.Cu") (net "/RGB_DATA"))
 (segment (start 104.03 114.65) (end 102.5 114.65) (width 0.25) (layer "F.Cu") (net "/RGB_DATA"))
 (segment (start 101.7 115.45) (end 101.7 140) (width 0.25) (layer "F.Cu") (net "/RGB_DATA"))
 (segment (start 101.7 140) (end 106.7 145) (width 0.25) (layer "F.Cu") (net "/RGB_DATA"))
 (segment (start 102.5 114.65) (end 101.7 115.45) (width 0.25) (layer "F.Cu") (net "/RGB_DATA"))
 (segment (start 129.9 145) (end 130.675 145) (width 0.25) (layer "F.Cu") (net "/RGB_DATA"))
 (segment (start 143 163.21) (end 129.8 163.21) (width 0.23) (layer "F.Cu") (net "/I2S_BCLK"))
 (segment (start 143 119.73) (end 143 148) (width 0.23) (layer "F.Cu") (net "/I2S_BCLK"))
 (segment (start 141.73 118.46) (end 143 119.73) (width 0.23) (layer "F.Cu") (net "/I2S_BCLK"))
 (segment (start 130.7 118.46) (end 141.73 118.46) (width 0.23) (layer "F.Cu") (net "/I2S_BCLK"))
 (segment (start 129.43 117.19) (end 130.7 118.46) (width 0.23) (layer "F.Cu") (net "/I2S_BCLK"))
 (segment (start 129.43 119.73) (end 130.7 121) (width 0.23) (layer "F.Cu") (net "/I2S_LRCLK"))
 (segment (start 130.7 121) (end 139.73 121) (width 0.23) (layer "F.Cu") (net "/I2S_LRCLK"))
 (segment (start 141 122.27) (end 141 148) (width 0.23) (layer "F.Cu") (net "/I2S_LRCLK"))
 (segment (start 141 165.21) (end 129.8 165.21) (width 0.23) (layer "F.Cu") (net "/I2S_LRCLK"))
 (segment (start 139.73 121) (end 141 122.27) (width 0.23) (layer "F.Cu") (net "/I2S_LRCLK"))
 (via (at 141 148) (size 0.65) (drill 0.3) (layers "F.Cu" "B.Cu") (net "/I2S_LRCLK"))
 (via (at 141 165.21) (size 0.65) (drill 0.3) (layers "F.Cu" "B.Cu") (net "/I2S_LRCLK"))
 (segment (start 137.73 123.54) (end 139 124.81) (width 0.23) (layer "F.Cu") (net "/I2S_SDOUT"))
 (segment (start 130.7 123.54) (end 137.73 123.54) (width 0.23) (layer "F.Cu") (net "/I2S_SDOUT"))
 (segment (start 129.43 122.27) (end 130.7 123.54) (width 0.23) (layer "F.Cu") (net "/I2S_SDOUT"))
 (segment (start 139 124.81) (end 139 148) (width 0.23) (layer "F.Cu") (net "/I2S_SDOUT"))
 (via (at 139 148) (size 0.65) (drill 0.3) (layers "F.Cu" "B.Cu") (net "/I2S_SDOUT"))
 (segment (start 137.6 154) (end 131.01 154) (width 0.23) (layer "B.Cu") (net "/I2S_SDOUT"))
 (segment (start 131.01 154) (end 129.8 155.21) (width 0.23) (layer "B.Cu") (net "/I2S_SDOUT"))
 (segment (start 139 148) (end 139 152.6) (width 0.23) (layer "B.Cu") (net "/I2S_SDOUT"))
 (segment (start 139 152.6) (end 137.6 154) (width 0.23) (layer "B.Cu") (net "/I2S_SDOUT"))
 (segment (start 143 148) (end 143 163.21) (width 0.23) (layer "F.Cu") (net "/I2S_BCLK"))
 (segment (start 141 148) (end 141 157.8) (width 0.23) (layer "B.Cu") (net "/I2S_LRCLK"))
 (via (at 141 157.8) (size 0.65) (drill 0.3) (layers "F.Cu" "B.Cu") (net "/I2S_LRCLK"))
 (segment (start 141 157.8) (end 141 162.2) (width 0.23) (layer "F.Cu") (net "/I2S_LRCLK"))
 (via (at 141 162.2) (size 0.65) (drill 0.3) (layers "F.Cu" "B.Cu") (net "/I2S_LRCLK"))
 (segment (start 141 162.2) (end 141 165.21) (width 0.23) (layer "B.Cu") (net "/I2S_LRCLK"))
 (segment (start 146.25 103.2) (end 140.67 103.2) (width 0.5) (layer "B.Cu") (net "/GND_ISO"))
 (segment (start 140.67 103.2) (end 134.3 109.57) (width 0.5) (layer "B.Cu") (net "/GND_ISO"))
 (segment (start 103.8 158.71) (end 107.1 158.71) (width 0.24) (layer "F.Cu") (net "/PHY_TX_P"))
 (segment (start 107.1 158.71) (end 107.1 164.555) (width 0.24) (layer "F.Cu") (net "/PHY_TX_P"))
 (segment (start 107.1 164.555) (end 108.745 164.555) (width 0.24) (layer "F.Cu") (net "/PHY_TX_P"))
 (segment (start 103.8 160.71) (end 106.5 160.71) (width 0.24) (layer "F.Cu") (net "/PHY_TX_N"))
 (segment (start 106.5 160.71) (end 106.5 167.095) (width 0.24) (layer "F.Cu") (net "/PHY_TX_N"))
 (segment (start 106.5 167.095) (end 108.745 167.095) (width 0.24) (layer "F.Cu") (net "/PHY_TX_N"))
 (segment (start 103.8 162.71) (end 105.9 162.71) (width 0.24) (layer "F.Cu") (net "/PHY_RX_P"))
 (segment (start 105.9 162.71) (end 105.9 170.905) (width 0.24) (layer "F.Cu") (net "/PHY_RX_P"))
 (segment (start 105.9 170.905) (end 108.745 170.905) (width 0.24) (layer "F.Cu") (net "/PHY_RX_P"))
 (segment (start 103.8 164.71) (end 105.3 164.71) (width 0.24) (layer "F.Cu") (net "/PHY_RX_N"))
 (segment (start 105.3 164.71) (end 105.3 173.445) (width 0.24) (layer "F.Cu") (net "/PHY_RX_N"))
 (segment (start 105.3 173.445) (end 108.745 173.445) (width 0.24) (layer "F.Cu") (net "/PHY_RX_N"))
 (segment (start 146.135 160) (end 144.865 160) (width 0.4) (layer "B.Cu") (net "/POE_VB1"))
 (segment (start 142.325 160) (end 141.055 160) (width 0.4) (layer "B.Cu") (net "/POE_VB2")))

